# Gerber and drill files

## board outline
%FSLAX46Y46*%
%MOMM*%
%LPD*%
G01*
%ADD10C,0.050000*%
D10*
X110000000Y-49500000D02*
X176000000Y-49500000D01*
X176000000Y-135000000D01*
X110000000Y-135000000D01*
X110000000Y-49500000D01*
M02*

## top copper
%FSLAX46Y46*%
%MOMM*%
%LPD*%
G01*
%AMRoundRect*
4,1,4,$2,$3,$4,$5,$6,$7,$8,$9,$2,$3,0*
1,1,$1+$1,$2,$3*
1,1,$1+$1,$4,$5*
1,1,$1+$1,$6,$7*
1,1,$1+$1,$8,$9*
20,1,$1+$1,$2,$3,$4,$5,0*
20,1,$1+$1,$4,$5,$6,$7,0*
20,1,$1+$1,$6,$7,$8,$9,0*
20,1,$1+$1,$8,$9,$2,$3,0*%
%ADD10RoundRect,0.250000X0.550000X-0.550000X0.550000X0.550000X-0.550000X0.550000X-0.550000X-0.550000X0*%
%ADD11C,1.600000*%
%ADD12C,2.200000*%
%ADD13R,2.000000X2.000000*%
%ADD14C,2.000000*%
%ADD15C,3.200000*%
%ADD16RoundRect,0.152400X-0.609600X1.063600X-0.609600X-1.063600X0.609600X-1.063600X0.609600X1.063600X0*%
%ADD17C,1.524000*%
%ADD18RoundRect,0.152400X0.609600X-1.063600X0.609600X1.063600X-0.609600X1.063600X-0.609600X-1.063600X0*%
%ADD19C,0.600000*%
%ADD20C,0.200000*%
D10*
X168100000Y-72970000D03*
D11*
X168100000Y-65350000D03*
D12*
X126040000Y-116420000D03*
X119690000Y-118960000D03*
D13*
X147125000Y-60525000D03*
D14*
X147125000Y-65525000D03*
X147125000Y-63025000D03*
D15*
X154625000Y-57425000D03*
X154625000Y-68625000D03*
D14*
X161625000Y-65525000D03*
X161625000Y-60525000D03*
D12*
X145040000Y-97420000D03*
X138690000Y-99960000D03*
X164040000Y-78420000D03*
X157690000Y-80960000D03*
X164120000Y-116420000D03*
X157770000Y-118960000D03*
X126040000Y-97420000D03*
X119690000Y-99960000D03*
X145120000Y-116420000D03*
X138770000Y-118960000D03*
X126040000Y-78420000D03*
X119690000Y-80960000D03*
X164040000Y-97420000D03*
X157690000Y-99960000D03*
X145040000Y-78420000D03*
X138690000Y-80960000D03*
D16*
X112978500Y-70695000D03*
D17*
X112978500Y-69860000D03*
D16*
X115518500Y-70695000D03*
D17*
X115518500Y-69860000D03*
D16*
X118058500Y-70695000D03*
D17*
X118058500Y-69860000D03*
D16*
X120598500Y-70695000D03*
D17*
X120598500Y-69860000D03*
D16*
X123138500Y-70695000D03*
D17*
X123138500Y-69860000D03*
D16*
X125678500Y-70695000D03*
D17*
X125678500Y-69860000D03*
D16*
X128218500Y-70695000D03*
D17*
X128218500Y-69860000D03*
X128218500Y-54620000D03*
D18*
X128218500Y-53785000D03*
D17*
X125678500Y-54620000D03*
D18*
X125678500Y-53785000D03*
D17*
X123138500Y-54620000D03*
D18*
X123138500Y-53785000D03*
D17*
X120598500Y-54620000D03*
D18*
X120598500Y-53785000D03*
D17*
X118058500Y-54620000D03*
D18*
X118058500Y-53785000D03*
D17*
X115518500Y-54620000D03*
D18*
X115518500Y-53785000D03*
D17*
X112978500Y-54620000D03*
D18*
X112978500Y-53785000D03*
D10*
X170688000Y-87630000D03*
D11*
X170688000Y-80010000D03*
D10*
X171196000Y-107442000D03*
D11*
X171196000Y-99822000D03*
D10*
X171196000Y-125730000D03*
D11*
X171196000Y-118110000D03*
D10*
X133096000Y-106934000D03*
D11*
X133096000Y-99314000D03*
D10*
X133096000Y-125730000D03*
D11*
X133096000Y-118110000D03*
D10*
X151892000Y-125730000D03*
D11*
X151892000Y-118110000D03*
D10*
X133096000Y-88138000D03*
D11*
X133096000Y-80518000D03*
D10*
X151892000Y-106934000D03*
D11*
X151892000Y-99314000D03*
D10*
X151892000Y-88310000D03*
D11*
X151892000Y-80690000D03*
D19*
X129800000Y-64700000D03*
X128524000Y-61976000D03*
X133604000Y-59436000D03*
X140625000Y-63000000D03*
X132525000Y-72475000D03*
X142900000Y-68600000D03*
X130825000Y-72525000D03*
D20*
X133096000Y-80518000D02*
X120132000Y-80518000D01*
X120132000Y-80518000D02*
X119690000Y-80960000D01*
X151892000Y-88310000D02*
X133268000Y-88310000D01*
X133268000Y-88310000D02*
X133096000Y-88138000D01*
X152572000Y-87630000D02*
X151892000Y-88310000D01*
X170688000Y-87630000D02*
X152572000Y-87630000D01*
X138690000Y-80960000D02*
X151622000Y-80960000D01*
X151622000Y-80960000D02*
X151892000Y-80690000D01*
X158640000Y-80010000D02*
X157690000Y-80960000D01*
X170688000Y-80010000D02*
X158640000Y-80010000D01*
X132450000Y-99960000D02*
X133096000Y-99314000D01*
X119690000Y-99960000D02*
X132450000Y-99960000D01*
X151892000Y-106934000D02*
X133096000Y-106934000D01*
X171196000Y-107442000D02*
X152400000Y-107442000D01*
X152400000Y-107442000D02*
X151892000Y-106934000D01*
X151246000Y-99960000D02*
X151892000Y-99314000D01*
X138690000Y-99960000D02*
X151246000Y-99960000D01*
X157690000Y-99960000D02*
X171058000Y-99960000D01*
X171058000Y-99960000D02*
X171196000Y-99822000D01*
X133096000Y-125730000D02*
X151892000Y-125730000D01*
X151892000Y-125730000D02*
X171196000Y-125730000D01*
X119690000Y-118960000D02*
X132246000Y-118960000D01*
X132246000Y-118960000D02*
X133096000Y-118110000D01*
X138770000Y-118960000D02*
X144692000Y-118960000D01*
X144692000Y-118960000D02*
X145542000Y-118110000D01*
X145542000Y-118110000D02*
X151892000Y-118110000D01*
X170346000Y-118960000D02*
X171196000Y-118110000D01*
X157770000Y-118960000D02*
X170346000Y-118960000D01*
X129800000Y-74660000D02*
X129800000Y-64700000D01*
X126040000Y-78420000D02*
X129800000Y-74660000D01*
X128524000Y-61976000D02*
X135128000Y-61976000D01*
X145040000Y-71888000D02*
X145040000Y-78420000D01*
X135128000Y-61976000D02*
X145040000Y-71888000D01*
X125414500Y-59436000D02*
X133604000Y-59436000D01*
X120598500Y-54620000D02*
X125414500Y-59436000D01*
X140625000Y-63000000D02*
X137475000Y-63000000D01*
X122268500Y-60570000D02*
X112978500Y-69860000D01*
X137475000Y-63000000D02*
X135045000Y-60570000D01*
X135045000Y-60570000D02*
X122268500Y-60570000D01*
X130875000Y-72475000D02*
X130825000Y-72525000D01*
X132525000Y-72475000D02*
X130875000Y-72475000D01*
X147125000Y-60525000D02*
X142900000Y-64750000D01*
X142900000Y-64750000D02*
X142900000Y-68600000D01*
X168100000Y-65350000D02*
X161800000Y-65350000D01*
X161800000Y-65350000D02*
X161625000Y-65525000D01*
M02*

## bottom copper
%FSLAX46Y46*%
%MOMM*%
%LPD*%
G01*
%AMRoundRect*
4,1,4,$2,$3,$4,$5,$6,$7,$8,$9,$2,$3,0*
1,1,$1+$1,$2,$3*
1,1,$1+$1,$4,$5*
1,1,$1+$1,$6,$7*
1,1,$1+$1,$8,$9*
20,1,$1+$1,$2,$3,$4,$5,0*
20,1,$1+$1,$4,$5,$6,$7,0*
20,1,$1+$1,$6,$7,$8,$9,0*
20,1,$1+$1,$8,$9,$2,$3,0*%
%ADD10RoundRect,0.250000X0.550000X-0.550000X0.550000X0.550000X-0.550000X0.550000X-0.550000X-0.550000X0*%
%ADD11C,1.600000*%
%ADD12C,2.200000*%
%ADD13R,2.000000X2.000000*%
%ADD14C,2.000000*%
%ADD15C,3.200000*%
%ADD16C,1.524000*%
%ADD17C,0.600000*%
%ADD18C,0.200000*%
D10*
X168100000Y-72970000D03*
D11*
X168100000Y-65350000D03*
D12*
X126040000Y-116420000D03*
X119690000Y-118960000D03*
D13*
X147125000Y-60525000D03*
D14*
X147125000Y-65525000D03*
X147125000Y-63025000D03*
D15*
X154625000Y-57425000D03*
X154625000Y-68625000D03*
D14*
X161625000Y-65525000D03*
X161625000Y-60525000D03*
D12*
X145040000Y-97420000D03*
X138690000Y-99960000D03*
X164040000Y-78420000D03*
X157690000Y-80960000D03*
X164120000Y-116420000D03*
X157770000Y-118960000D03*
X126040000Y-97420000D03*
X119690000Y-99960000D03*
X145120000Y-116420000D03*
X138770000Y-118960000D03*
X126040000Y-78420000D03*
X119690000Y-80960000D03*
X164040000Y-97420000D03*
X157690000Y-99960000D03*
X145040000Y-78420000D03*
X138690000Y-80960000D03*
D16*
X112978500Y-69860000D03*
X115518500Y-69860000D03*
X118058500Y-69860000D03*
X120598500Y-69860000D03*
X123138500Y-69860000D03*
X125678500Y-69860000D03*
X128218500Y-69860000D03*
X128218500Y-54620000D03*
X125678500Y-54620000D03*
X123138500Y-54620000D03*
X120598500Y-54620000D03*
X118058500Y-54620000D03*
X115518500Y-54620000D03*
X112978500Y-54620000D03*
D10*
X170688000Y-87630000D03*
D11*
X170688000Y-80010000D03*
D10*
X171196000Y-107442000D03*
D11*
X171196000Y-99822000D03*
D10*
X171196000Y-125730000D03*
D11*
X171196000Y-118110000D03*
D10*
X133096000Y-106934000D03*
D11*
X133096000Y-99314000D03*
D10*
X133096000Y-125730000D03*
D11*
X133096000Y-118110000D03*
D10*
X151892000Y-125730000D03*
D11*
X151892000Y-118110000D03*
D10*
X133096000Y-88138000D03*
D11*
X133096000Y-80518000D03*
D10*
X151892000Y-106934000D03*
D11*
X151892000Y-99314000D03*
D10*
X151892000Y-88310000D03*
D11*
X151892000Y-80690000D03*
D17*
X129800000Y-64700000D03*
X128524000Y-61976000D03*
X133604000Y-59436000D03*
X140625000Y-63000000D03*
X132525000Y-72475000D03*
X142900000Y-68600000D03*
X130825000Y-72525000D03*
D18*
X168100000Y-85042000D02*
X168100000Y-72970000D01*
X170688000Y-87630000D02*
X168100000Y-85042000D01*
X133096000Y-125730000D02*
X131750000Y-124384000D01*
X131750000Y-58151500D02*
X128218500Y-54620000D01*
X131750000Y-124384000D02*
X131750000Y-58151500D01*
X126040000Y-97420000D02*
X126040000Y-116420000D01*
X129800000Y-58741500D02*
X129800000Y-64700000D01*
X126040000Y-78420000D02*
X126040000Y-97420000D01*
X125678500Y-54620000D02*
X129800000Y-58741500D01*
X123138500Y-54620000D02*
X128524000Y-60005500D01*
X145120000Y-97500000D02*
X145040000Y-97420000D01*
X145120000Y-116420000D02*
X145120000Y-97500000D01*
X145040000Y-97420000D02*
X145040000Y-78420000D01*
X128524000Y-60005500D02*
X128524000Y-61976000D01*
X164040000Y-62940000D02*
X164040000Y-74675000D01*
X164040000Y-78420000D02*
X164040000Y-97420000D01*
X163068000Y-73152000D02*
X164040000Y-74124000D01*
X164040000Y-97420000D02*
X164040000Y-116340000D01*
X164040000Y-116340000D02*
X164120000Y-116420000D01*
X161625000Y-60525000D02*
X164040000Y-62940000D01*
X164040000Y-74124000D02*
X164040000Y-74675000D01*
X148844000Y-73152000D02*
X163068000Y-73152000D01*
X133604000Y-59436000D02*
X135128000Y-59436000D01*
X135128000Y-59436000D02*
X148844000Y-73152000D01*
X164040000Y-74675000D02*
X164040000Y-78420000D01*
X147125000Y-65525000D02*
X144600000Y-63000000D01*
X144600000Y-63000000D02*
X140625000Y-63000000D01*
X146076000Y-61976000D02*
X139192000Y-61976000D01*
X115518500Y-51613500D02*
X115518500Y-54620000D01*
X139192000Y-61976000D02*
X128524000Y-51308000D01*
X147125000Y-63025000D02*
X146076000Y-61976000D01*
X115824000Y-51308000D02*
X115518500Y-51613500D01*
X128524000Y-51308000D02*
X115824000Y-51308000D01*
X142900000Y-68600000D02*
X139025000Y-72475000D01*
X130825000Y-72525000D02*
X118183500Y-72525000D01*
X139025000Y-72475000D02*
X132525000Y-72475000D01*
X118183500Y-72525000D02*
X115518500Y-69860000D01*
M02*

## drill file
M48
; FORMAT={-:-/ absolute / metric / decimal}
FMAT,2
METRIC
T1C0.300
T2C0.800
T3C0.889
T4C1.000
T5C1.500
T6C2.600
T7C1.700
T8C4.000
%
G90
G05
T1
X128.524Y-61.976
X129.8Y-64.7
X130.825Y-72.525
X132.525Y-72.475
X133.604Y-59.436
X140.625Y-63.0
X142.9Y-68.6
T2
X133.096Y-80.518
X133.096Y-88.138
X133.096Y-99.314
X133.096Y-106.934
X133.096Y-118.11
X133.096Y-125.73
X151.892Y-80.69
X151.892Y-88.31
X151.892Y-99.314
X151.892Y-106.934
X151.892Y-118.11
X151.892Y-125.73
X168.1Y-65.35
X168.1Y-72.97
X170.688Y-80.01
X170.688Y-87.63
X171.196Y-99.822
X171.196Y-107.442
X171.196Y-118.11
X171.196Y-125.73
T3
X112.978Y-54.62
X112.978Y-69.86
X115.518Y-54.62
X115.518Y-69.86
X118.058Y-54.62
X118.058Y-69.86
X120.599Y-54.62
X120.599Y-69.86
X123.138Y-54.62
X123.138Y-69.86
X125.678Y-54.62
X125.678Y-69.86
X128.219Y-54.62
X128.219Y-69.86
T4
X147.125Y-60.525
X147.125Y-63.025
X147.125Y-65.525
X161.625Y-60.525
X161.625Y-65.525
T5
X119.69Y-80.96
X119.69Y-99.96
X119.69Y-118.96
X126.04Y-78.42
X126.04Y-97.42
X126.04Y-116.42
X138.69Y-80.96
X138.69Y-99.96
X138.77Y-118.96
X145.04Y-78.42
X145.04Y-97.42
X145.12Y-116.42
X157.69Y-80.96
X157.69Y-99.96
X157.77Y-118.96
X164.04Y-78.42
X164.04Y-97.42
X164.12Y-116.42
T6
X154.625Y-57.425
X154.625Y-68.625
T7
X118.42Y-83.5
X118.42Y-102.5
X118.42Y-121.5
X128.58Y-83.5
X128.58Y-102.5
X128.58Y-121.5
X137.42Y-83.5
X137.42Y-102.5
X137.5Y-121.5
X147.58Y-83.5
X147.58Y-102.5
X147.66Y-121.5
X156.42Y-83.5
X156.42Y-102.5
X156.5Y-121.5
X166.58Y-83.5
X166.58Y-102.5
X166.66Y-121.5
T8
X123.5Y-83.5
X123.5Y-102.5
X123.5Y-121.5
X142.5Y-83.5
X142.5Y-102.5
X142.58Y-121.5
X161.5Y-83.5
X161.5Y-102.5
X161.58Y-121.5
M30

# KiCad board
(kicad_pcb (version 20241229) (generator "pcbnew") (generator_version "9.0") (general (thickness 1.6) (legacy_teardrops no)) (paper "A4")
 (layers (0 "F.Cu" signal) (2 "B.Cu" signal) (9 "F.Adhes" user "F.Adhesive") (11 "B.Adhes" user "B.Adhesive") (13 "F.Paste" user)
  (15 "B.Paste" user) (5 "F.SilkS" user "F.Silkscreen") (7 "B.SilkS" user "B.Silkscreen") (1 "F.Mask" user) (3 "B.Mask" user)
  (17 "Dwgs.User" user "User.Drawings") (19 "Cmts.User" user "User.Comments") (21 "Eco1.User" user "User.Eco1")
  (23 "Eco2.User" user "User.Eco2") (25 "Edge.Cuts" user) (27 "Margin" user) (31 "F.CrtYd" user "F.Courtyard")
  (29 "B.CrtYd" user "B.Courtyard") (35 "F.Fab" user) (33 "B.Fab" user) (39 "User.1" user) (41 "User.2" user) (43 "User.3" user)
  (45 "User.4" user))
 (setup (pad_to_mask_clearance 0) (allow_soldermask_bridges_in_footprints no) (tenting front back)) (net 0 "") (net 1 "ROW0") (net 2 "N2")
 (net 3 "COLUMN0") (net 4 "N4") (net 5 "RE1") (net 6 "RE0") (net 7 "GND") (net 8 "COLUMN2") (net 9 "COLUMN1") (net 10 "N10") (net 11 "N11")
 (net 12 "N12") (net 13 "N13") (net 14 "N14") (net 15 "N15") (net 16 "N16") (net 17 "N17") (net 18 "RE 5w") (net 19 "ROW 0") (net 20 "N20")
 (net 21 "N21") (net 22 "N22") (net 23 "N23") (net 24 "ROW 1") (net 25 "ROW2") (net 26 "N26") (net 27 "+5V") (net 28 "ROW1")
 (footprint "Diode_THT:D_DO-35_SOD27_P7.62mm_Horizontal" (layer "F.Cu") (at 168.1 72.97 90)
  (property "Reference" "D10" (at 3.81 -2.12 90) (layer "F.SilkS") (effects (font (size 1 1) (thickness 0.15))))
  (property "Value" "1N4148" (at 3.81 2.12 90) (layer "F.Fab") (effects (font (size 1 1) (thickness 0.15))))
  (pad "1" thru_hole roundrect (at 0 0 90) (size 1.6 1.6) (drill 0.8) (layers "*.Cu" "*.Mask") (remove_unused_layers no)
   (roundrect_rratio 0.15625) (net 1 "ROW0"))
  (pad "2" thru_hole circle (at 7.62 0 90) (size 1.6 1.6) (drill 0.8) (layers "*.Cu" "*.Mask") (remove_unused_layers no) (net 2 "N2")))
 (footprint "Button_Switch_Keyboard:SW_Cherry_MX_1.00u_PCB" (layer "F.Cu") (at 126.04 116.42)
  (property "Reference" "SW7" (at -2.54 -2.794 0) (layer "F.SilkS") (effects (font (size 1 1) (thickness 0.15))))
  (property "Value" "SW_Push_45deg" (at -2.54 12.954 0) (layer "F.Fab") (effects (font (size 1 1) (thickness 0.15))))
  (pad "" np_thru_hole circle (at -7.62 5.08) (size 1.7 1.7) (drill 1.7) (layers "*.Cu" "*.Mask"))
  (pad "" np_thru_hole circle (at -2.54 5.08) (size 4 4) (drill 4) (layers "*.Cu" "*.Mask"))
  (pad "" np_thru_hole circle (at 2.54 5.08) (size 1.7 1.7) (drill 1.7) (layers "*.Cu" "*.Mask"))
  (pad "1" thru_hole circle (at 0 0) (size 2.2 2.2) (drill 1.5) (layers "*.Cu" "*.Mask") (remove_unused_layers no) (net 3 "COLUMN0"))
  (pad "2" thru_hole circle (at -6.35 2.54) (size 2.2 2.2) (drill 1.5) (layers "*.Cu" "*.Mask") (remove_unused_layers no) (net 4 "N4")))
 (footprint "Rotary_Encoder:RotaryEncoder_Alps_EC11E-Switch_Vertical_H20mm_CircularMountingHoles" (layer "F.Cu") (at 147.125 60.525)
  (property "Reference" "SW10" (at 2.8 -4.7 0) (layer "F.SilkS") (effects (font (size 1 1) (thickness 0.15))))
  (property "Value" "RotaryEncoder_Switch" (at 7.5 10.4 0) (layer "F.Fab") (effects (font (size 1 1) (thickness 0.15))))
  (pad "A" thru_hole rect (at 0 0) (size 2 2) (drill 1) (layers "*.Cu" "*.Mask") (remove_unused_layers no) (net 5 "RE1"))
  (pad "B" thru_hole circle (at 0 5) (size 2 2) (drill 1) (layers "*.Cu" "*.Mask") (remove_unused_layers no) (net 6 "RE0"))
  (pad "C" thru_hole circle (at 0 2.5) (size 2 2) (drill 1) (layers "*.Cu" "*.Mask") (remove_unused_layers no) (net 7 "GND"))
  (pad "MP" thru_hole circle (at 7.5 -3.1) (size 3.2 3.2) (drill 2.6) (layers "*.Cu" "*.Mask") (remove_unused_layers no))
  (pad "MP" thru_hole circle (at 7.5 8.1) (size 3.2 3.2) (drill 2.6) (layers "*.Cu" "*.Mask") (remove_unused_layers no))
  (pad "S1" thru_hole circle (at 14.5 5) (size 2 2) (drill 1) (layers "*.Cu" "*.Mask") (remove_unused_layers no) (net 2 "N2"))
  (pad "S2" thru_hole circle (at 14.5 0) (size 2 2) (drill 1) (layers "*.Cu" "*.Mask") (remove_unused_layers no) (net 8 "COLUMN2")))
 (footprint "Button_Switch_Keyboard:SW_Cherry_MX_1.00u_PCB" (layer "F.Cu") (at 145.04 97.42)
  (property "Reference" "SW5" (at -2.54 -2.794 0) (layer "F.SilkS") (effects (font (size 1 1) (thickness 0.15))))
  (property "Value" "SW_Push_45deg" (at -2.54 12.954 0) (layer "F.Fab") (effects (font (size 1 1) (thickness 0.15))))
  (pad "" np_thru_hole circle (at -7.62 5.08) (size 1.7 1.7) (drill 1.7) (layers "*.Cu" "*.Mask"))
  (pad "" np_thru_hole circle (at -2.54 5.08) (size 4 4) (drill 4) (layers "*.Cu" "*.Mask"))
  (pad "" np_thru_hole circle (at 2.54 5.08) (size 1.7 1.7) (drill 1.7) (layers "*.Cu" "*.Mask"))
  (pad "1" thru_hole circle (at 0 0) (size 2.2 2.2) (drill 1.5) (layers "*.Cu" "*.Mask") (remove_unused_layers no) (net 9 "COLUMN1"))
  (pad "2" thru_hole circle (at -6.35 2.54) (size 2.2 2.2) (drill 1.5) (layers "*.Cu" "*.Mask") (remove_unused_layers no) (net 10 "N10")))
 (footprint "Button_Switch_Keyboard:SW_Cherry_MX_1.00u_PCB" (layer "F.Cu") (at 164.04 78.42)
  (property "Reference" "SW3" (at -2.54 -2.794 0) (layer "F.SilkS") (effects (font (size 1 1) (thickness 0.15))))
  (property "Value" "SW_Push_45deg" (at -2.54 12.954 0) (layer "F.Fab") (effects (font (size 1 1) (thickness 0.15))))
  (pad "" np_thru_hole circle (at -7.62 5.08) (size 1.7 1.7) (drill 1.7) (layers "*.Cu" "*.Mask"))
  (pad "" np_thru_hole circle (at -2.54 5.08) (size 4 4) (drill 4) (layers "*.Cu" "*.Mask"))
  (pad "" np_thru_hole circle (at 2.54 5.08) (size 1.7 1.7) (drill 1.7) (layers "*.Cu" "*.Mask"))
  (pad "1" thru_hole circle (at 0 0) (size 2.2 2.2) (drill 1.5) (layers "*.Cu" "*.Mask") (remove_unused_layers no) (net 8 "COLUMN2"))
  (pad "2" thru_hole circle (at -6.35 2.54) (size 2.2 2.2) (drill 1.5) (layers "*.Cu" "*.Mask") (remove_unused_layers no) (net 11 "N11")))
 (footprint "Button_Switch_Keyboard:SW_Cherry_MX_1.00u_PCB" (layer "F.Cu") (at 164.12 116.42)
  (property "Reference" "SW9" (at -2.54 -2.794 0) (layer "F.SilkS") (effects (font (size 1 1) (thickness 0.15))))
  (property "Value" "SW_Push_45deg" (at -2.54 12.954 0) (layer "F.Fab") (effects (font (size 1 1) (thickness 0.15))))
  (pad "" np_thru_hole circle (at -7.62 5.08) (size 1.7 1.7) (drill 1.7) (layers "*.Cu" "*.Mask"))
  (pad "" np_thru_hole circle (at -2.54 5.08) (size 4 4) (drill 4) (layers "*.Cu" "*.Mask"))
  (pad "" np_thru_hole circle (at 2.54 5.08) (size 1.7 1.7) (drill 1.7) (layers "*.Cu" "*.Mask"))
  (pad "1" thru_hole circle (at 0 0) (size 2.2 2.2) (drill 1.5) (layers "*.Cu" "*.Mask") (remove_unused_layers no) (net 8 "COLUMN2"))
  (pad "2" thru_hole circle (at -6.35 2.54) (size 2.2 2.2) (drill 1.5) (layers "*.Cu" "*.Mask") (remove_unused_layers no) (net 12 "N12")))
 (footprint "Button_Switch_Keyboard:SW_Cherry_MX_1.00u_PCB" (layer "F.Cu") (at 126.04 97.42)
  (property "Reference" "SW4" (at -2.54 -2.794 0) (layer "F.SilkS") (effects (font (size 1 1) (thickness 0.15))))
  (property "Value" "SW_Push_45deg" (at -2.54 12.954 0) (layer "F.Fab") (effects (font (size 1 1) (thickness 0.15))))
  (pad "" np_thru_hole circle (at -7.62 5.08) (size 1.7 1.7) (drill 1.7) (layers "*.Cu" "*.Mask"))
  (pad "" np_thru_hole circle (at -2.54 5.08) (size 4 4) (drill 4) (layers "*.Cu" "*.Mask"))
  (pad "" np_thru_hole circle (at 2.54 5.08) (size 1.7 1.7) (drill 1.7) (layers "*.Cu" "*.Mask"))
  (pad "1" thru_hole circle (at 0 0) (size 2.2 2.2) (drill 1.5) (layers "*.Cu" "*.Mask") (remove_unused_layers no) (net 3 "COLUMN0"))
  (pad "2" thru_hole circle (at -6.35 2.54) (size 2.2 2.2) (drill 1.5) (layers "*.Cu" "*.Mask") (remove_unused_layers no) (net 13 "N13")))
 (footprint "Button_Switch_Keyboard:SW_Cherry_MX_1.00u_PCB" (layer "F.Cu") (at 145.12 116.42)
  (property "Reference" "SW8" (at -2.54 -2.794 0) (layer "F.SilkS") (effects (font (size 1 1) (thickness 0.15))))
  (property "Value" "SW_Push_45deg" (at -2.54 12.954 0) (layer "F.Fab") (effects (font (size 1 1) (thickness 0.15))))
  (pad "" np_thru_hole circle (at -7.62 5.08) (size 1.7 1.7) (drill 1.7) (layers "*.Cu" "*.Mask"))
  (pad "" np_thru_hole circle (at -2.54 5.08) (size 4 4) (drill 4) (layers "*.Cu" "*.Mask"))
  (pad "" np_thru_hole circle (at 2.54 5.08) (size 1.7 1.7) (drill 1.7) (layers "*.Cu" "*.Mask"))
  (pad "1" thru_hole circle (at 0 0) (size 2.2 2.2) (drill 1.5) (layers "*.Cu" "*.Mask") (remove_unused_layers no) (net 9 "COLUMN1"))
  (pad "2" thru_hole circle (at -6.35 2.54) (size 2.2 2.2) (drill 1.5) (layers "*.Cu" "*.Mask") (remove_unused_layers no) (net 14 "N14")))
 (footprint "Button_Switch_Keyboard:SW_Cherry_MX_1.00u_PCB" (layer "F.Cu") (at 126.04 78.42)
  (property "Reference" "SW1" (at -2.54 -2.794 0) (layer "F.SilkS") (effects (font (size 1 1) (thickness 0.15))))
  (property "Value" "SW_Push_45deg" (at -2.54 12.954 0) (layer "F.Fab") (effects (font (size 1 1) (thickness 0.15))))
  (pad "" np_thru_hole circle (at -7.62 5.08) (size 1.7 1.7) (drill 1.7) (layers "*.Cu" "*.Mask"))
  (pad "" np_thru_hole circle (at -2.54 5.08) (size 4 4) (drill 4) (layers "*.Cu" "*.Mask"))
  (pad "" np_thru_hole circle (at 2.54 5.08) (size 1.7 1.7) (drill 1.7) (layers "*.Cu" "*.Mask"))
  (pad "1" thru_hole circle (at 0 0) (size 2.2 2.2) (drill 1.5) (layers "*.Cu" "*.Mask") (remove_unused_layers no) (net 3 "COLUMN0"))
  (pad "2" thru_hole circle (at -6.35 2.54) (size 2.2 2.2) (drill 1.5) (layers "*.Cu" "*.Mask") (remove_unused_layers no) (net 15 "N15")))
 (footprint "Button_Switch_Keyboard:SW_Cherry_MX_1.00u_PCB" (layer "F.Cu") (at 164.04 97.42)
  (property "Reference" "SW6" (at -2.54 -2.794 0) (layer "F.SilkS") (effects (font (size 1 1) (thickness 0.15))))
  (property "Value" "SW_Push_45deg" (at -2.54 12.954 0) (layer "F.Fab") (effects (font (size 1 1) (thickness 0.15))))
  (pad "" np_thru_hole circle (at -7.62 5.08) (size 1.7 1.7) (drill 1.7) (layers "*.Cu" "*.Mask"))
  (pad "" np_thru_hole circle (at -2.54 5.08) (size 4 4) (drill 4) (layers "*.Cu" "*.Mask"))
  (pad "" np_thru_hole circle (at 2.54 5.08) (size 1.7 1.7) (drill 1.7) (layers "*.Cu" "*.Mask"))
  (pad "1" thru_hole circle (at 0 0) (size 2.2 2.2) (drill 1.5) (layers "*.Cu" "*.Mask") (remove_unused_layers no) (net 8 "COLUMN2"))
  (pad "2" thru_hole circle (at -6.35 2.54) (size 2.2 2.2) (drill 1.5) (layers "*.Cu" "*.Mask") (remove_unused_layers no) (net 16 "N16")))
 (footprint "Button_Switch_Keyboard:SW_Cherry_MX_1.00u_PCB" (layer "F.Cu") (at 145.04 78.42)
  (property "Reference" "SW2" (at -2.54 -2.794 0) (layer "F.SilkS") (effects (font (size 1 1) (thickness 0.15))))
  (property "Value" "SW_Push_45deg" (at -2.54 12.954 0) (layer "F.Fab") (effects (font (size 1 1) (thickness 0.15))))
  (pad "" np_thru_hole circle (at -7.62 5.08) (size 1.7 1.7) (drill 1.7) (layers "*.Cu" "*.Mask"))
  (pad "" np_thru_hole circle (at -2.54 5.08) (size 4 4) (drill 4) (layers "*.Cu" "*.Mask"))
  (pad "" np_thru_hole circle (at 2.54 5.08) (size 1.7 1.7) (drill 1.7) (layers "*.Cu" "*.Mask"))
  (pad "1" thru_hole circle (at 0 0) (size 2.2 2.2) (drill 1.5) (layers "*.Cu" "*.Mask") (remove_unused_layers no) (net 9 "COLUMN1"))
  (pad "2" thru_hole circle (at -6.35 2.54) (size 2.2 2.2) (drill 1.5) (layers "*.Cu" "*.Mask") (remove_unused_layers no) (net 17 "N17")))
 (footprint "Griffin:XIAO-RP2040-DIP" (layer "F.Cu") (at 120.5985 62.24 90)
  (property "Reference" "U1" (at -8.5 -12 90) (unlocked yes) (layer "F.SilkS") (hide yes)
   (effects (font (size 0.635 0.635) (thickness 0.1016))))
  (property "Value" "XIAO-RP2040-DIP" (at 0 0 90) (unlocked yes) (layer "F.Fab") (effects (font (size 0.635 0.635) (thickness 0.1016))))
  (pad "1" smd roundrect (at -8.455 -7.62 270) (size 2.432 1.524) (layers "F.Cu" "F.Mask") (roundrect_rratio 0.1) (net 6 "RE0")
   (thermal_bridge_angle 45))
  (pad "1" thru_hole circle (at -7.62 -7.62 270) (size 1.524 1.524) (drill 0.889) (layers "*.Cu" "*.Mask") (remove_unused_layers no)
   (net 6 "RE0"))
  (pad "2" smd roundrect (at -8.455 -5.08 270) (size 2.432 1.524) (layers "F.Cu" "F.Mask") (roundrect_rratio 0.1) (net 5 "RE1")
   (thermal_bridge_angle 45))
  (pad "2" thru_hole circle (at -7.62 -5.08 270) (size 1.524 1.524) (drill 0.889) (layers "*.Cu" "*.Mask") (remove_unused_layers no)
   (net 5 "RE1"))
  (pad "3" smd roundrect (at -8.455 -2.54 270) (size 2.432 1.524) (layers "F.Cu" "F.Mask") (roundrect_rratio 0.1) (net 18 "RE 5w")
   (thermal_bridge_angle 45))
  (pad "3" thru_hole circle (at -7.62 -2.54 270) (size 1.524 1.524) (drill 0.889) (layers "*.Cu" "*.Mask") (remove_unused_layers no)
   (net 18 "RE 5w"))
  (pad "4" smd roundrect (at -8.455 0 270) (size 2.432 1.524) (layers "F.Cu" "F.Mask") (roundrect_rratio 0.1) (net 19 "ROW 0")
   (thermal_bridge_angle 45))
  (pad "4" thru_hole circle (at -7.62 0 270) (size 1.524 1.524) (drill 0.889) (layers "*.Cu" "*.Mask") (remove_unused_layers no)
   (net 19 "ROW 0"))
  (pad "5" smd roundrect (at -8.455 2.54 270) (size 2.432 1.524) (layers "F.Cu" "F.Mask") (roundrect_rratio 0.1) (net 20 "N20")
   (thermal_bridge_angle 45))
  (pad "5" thru_hole circle (at -7.62 2.54 270) (size 1.524 1.524) (drill 0.889) (layers "*.Cu" "*.Mask") (remove_unused_layers no)
   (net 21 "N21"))
  (pad "6" smd roundrect (at -8.455 5.08 270) (size 2.432 1.524) (layers "F.Cu" "F.Mask") (roundrect_rratio 0.1) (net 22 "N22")
   (thermal_bridge_angle 45))
  (pad "6" thru_hole circle (at -7.62 5.08 270) (size 1.524 1.524) (drill 0.889) (layers "*.Cu" "*.Mask") (remove_unused_layers no)
   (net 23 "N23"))
  (pad "7" smd roundrect (at -8.455 7.62 270) (size 2.432 1.524) (layers "F.Cu" "F.Mask") (roundrect_rratio 0.1) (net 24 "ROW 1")
   (thermal_bridge_angle 45))
  (pad "7" thru_hole circle (at -7.62 7.62 270) (size 1.524 1.524) (drill 0.889) (layers "*.Cu" "*.Mask") (remove_unused_layers no)
   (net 24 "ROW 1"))
  (pad "8" thru_hole circle (at 7.62 7.62 90) (size 1.524 1.524) (drill 0.889) (layers "*.Cu" "*.Mask") (remove_unused_layers no)
   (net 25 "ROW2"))
  (pad "8" smd roundrect (at 8.455 7.62 90) (size 2.432 1.524) (layers "F.Cu" "F.Mask") (roundrect_rratio 0.1) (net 25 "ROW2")
   (thermal_bridge_angle 45))
  (pad "9" thru_hole circle (at 7.62 5.08 90) (size 1.524 1.524) (drill 0.889) (layers "*.Cu" "*.Mask") (remove_unused_layers no)
   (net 3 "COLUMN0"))
  (pad "9" smd roundrect (at 8.455 5.08 90) (size 2.432 1.524) (layers "F.Cu" "F.Mask") (roundrect_rratio 0.1) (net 3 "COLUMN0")
   (thermal_bridge_angle 45))
  (pad "10" thru_hole circle (at 7.62 2.54 90) (size 1.524 1.524) (drill 0.889) (layers "*.Cu" "*.Mask") (remove_unused_layers no)
   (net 9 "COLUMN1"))
  (pad "10" smd roundrect (at 8.455 2.54 90) (size 2.432 1.524) (layers "F.Cu" "F.Mask") (roundrect_rratio 0.1) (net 9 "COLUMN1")
   (thermal_bridge_angle 45))
  (pad "11" thru_hole circle (at 7.62 0 90) (size 1.524 1.524) (drill 0.889) (layers "*.Cu" "*.Mask") (remove_unused_layers no)
   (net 8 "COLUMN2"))
  (pad "11" smd roundrect (at 8.455 0 90) (size 2.432 1.524) (layers "F.Cu" "F.Mask") (roundrect_rratio 0.1) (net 8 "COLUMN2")
   (thermal_bridge_angle 45))
  (pad "12" thru_hole circle (at 7.62 -2.54 90) (size 1.524 1.524) (drill 0.889) (layers "*.Cu" "*.Mask") (remove_unused_layers no)
   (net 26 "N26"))
  (pad "12" smd roundrect (at 8.455 -2.54 90) (size 2.432 1.524) (layers "F.Cu" "F.Mask") (roundrect_rratio 0.1) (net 26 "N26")
   (thermal_bridge_angle 45))
  (pad "13" thru_hole circle (at 7.62 -5.08 90) (size 1.524 1.524) (drill 0.889) (layers "*.Cu" "*.Mask") (remove_unused_layers no)
   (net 7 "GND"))
  (pad "13" smd roundrect (at 8.455 -5.08 90) (size 2.432 1.524) (layers "F.Cu" "F.Mask") (roundrect_rratio 0.1) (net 7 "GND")
   (thermal_bridge_angle 45))
  (pad "14" thru_hole circle (at 7.62 -7.62 90) (size 1.524 1.524) (drill 0.889) (layers "*.Cu" "*.Mask") (remove_unused_layers no)
   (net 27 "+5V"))
  (pad "14" smd roundrect (at 8.455 -7.62 90) (size 2.432 1.524) (layers "F.Cu" "F.Mask") (roundrect_rratio 0.1) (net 27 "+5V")
   (thermal_bridge_angle 45)))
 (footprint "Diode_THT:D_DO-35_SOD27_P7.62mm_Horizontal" (layer "B.Cu") (at 170.688 87.63 90)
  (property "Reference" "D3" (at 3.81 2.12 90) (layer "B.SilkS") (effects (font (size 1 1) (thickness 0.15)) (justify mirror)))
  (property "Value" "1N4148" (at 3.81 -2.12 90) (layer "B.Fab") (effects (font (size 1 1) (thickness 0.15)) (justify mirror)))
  (pad "1" thru_hole roundrect (at 0 0 90) (size 1.6 1.6) (drill 0.8) (layers "*.Cu" "*.Mask") (remove_unused_layers no)
   (roundrect_rratio 0.15625) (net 1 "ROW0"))
  (pad "2" thru_hole circle (at 7.62 0 90) (size 1.6 1.6) (drill 0.8) (layers "*.Cu" "*.Mask") (remove_unused_layers no) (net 11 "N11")))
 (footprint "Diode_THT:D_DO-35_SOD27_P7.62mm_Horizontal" (layer "B.Cu") (at 171.196 107.442 90)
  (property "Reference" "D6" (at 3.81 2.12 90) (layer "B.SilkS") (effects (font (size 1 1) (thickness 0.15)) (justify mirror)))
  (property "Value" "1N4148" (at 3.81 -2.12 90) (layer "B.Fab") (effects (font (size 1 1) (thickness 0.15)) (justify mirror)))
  (pad "1" thru_hole roundrect (at 0 0 90) (size 1.6 1.6) (drill 0.8) (layers "*.Cu" "*.Mask") (remove_unused_layers no)
   (roundrect_rratio 0.15625) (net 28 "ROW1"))
  (pad "2" thru_hole circle (at 7.62 0 90) (size 1.6 1.6) (drill 0.8) (layers "*.Cu" "*.Mask") (remove_unused_layers no) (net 16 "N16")))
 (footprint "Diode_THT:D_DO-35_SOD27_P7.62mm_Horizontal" (layer "B.Cu") (at 171.196 125.73 90)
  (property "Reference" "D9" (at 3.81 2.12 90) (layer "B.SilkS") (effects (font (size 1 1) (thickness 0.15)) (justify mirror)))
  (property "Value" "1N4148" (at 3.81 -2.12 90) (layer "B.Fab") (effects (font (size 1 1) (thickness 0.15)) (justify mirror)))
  (pad "1" thru_hole roundrect (at 0 0 90) (size 1.6 1.6) (drill 0.8) (layers "*.Cu" "*.Mask") (remove_unused_layers no)
   (roundrect_rratio 0.15625) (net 25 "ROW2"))
  (pad "2" thru_hole circle (at 7.62 0 90) (size 1.6 1.6) (drill 0.8) (layers "*.Cu" "*.Mask") (remove_unused_layers no) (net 12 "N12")))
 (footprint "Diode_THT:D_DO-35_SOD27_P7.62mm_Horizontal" (layer "B.Cu") (at 133.096 106.934 90)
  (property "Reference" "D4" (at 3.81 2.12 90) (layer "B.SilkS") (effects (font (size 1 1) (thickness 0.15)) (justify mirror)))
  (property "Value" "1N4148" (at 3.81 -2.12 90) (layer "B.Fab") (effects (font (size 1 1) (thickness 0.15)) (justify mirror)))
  (pad "1" thru_hole roundrect (at 0 0 90) (size 1.6 1.6) (drill 0.8) (layers "*.Cu" "*.Mask") (remove_unused_layers no)
   (roundrect_rratio 0.15625) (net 28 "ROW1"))
  (pad "2" thru_hole circle (at 7.62 0 90) (size 1.6 1.6) (drill 0.8) (layers "*.Cu" "*.Mask") (remove_unused_layers no) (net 13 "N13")))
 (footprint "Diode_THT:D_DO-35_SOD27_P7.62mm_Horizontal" (layer "B.Cu") (at 133.096 125.73 90)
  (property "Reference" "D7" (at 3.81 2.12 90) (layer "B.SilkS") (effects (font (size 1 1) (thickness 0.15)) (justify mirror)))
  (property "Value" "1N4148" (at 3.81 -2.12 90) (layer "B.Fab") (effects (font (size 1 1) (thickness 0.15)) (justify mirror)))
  (pad "1" thru_hole roundrect (at 0 0 90) (size 1.6 1.6) (drill 0.8) (layers "*.Cu" "*.Mask") (remove_unused_layers no)
   (roundrect_rratio 0.15625) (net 25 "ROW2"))
  (pad "2" thru_hole circle (at 7.62 0 90) (size 1.6 1.6) (drill 0.8) (layers "*.Cu" "*.Mask") (remove_unused_layers no) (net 4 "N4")))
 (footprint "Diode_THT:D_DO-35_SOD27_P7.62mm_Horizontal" (layer "B.Cu") (at 151.892 125.73 90)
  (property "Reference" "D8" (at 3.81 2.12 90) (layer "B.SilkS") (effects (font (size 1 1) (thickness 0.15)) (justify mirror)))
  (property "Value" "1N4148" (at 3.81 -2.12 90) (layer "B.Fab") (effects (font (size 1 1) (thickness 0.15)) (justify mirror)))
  (pad "1" thru_hole roundrect (at 0 0 90) (size 1.6 1.6) (drill 0.8) (layers "*.Cu" "*.Mask") (remove_unused_layers no)
   (roundrect_rratio 0.15625) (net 25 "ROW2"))
  (pad "2" thru_hole circle (at 7.62 0 90) (size 1.6 1.6) (drill 0.8) (layers "*.Cu" "*.Mask") (remove_unused_layers no) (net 14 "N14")))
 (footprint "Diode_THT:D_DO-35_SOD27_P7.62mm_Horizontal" (layer "B.Cu") (at 133.096 88.138 90)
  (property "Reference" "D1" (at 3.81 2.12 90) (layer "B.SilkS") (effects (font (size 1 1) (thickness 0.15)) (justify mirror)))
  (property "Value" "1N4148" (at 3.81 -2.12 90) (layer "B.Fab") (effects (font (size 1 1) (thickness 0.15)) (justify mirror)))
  (pad "1" thru_hole roundrect (at 0 0 90) (size 1.6 1.6) (drill 0.8) (layers "*.Cu" "*.Mask") (remove_unused_layers no)
   (roundrect_rratio 0.15625) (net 1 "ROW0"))
  (pad "2" thru_hole circle (at 7.62 0 90) (size 1.6 1.6) (drill 0.8) (layers "*.Cu" "*.Mask") (remove_unused_layers no) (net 15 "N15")))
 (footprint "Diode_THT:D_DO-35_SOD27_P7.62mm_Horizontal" (layer "B.Cu") (at 151.892 106.934 90)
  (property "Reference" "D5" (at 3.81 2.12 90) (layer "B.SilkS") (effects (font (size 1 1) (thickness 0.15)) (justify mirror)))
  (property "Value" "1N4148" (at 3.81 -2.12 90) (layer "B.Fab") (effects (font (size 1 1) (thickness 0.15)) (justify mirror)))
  (pad "1" thru_hole roundrect (at 0 0 90) (size 1.6 1.6) (drill 0.8) (layers "*.Cu" "*.Mask") (remove_unused_layers no)
   (roundrect_rratio 0.15625) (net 28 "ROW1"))
  (pad "2" thru_hole circle (at 7.62 0 90) (size 1.6 1.6) (drill 0.8) (layers "*.Cu" "*.Mask") (remove_unused_layers no) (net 10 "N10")))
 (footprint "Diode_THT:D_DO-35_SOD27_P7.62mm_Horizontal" (layer "B.Cu") (at 151.892 88.31 90)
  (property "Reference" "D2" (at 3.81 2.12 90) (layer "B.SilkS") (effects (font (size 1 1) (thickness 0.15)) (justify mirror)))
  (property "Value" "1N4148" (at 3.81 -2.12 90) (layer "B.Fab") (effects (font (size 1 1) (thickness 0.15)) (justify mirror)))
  (pad "1" thru_hole roundrect (at 0 0 90) (size 1.6 1.6) (drill 0.8) (layers "*.Cu" "*.Mask") (remove_unused_layers no)
   (roundrect_rratio 0.15625) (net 1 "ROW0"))
  (pad "2" thru_hole circle (at 7.62 0 90) (size 1.6 1.6) (drill 0.8) (layers "*.Cu" "*.Mask") (remove_unused_layers no) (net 17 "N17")))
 (gr_rect (start 110 49.5) (end 176 135) (stroke (width 0.05) (type default)) (fill no) (layer "Edge.Cuts"))
 (segment (start 133.096 80.518) (end 120.132 80.518) (width 0.2) (layer "F.Cu") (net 15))
 (segment (start 120.132 80.518) (end 119.69 80.96) (width 0.2) (layer "F.Cu") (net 15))
 (segment (start 151.892 88.31) (end 133.268 88.31) (width 0.2) (layer "F.Cu") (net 1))
 (segment (start 133.268 88.31) (end 133.096 88.138) (width 0.2) (layer "F.Cu") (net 1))
 (segment (start 152.572 87.63) (end 151.892 88.31) (width 0.2) (layer "F.Cu") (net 1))
 (segment (start 170.688 87.63) (end 152.572 87.63) (width 0.2) (layer "F.Cu") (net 1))
 (segment (start 168.1 85.042) (end 168.1 72.97) (width 0.2) (layer "B.Cu") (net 1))
 (segment (start 170.688 87.63) (end 168.1 85.042) (width 0.2) (layer "B.Cu") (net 1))
 (segment (start 138.69 80.96) (end 151.622 80.96) (width 0.2) (layer "F.Cu") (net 17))
 (segment (start 151.622 80.96) (end 151.892 80.69) (width 0.2) (layer "F.Cu") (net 17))
 (segment (start 158.64 80.01) (end 157.69 80.96) (width 0.2) (layer "F.Cu") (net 11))
 (segment (start 170.688 80.01) (end 158.64 80.01) (width 0.2) (layer "F.Cu") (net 11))
 (segment (start 132.45 99.96) (end 133.096 99.314) (width 0.2) (layer "F.Cu") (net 13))
 (segment (start 119.69 99.96) (end 132.45 99.96) (width 0.2) (layer "F.Cu") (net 13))
 (segment (start 151.892 106.934) (end 133.096 106.934) (width 0.2) (layer "F.Cu") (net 28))
 (segment (start 171.196 107.442) (end 152.4 107.442) (width 0.2) (layer "F.Cu") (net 28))
 (segment (start 152.4 107.442) (end 151.892 106.934) (width 0.2) (layer "F.Cu") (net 28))
 (segment (start 151.246 99.96) (end 151.892 99.314) (width 0.2) (layer "F.Cu") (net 10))
 (segment (start 138.69 99.96) (end 151.246 99.96) (width 0.2) (layer "F.Cu") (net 10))
 (segment (start 157.69 99.96) (end 171.058 99.96) (width 0.2) (layer "F.Cu") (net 16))
 (segment (start 171.058 99.96) (end 171.196 99.822) (width 0.2) (layer "F.Cu") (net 16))
 (segment (start 133.096 125.73) (end 151.892 125.73) (width 0.2) (layer "F.Cu") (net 25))
 (segment (start 151.892 125.73) (end 171.196 125.73) (width 0.2) (layer "F.Cu") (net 25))
 (segment (start 133.096 125.73) (end 131.75 124.384) (width 0.2) (layer "B.Cu") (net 25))
 (segment (start 131.75 58.1515) (end 128.2185 54.62) (width 0.2) (layer "B.Cu") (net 25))
 (segment (start 131.75 124.384) (end 131.75 58.1515) (width 0.2) (layer "B.Cu") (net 25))
 (segment (start 119.69 118.96) (end 132.246 118.96) (width 0.2) (layer "F.Cu") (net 4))
 (segment (start 132.246 118.96) (end 133.096 118.11) (width 0.2) (layer "F.Cu") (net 4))
 (segment (start 138.77 118.96) (end 144.692 118.96) (width 0.2) (layer "F.Cu") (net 14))
 (segment (start 144.692 118.96) (end 145.542 118.11) (width 0.2) (layer "F.Cu") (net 14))
 (segment (start 145.542 118.11) (end 151.892 118.11) (width 0.2) (layer "F.Cu") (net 14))
 (segment (start 170.346 118.96) (end 171.196 118.11) (width 0.2) (layer "F.Cu") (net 12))
 (segment (start 157.77 118.96) (end 170.346 118.96) (width 0.2) (layer "F.Cu") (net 12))
 (segment (start 129.8 74.66) (end 129.8 64.7) (width 0.2) (layer "F.Cu") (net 3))
 (segment (start 126.04 78.42) (end 129.8 74.66) (width 0.2) (layer "F.Cu") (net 3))
 (via (at 129.8 64.7) (size 0.6) (drill 0.3) (layers "F.Cu" "B.Cu") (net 3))
 (segment (start 126.04 97.42) (end 126.04 116.42) (width 0.2) (layer "B.Cu") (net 3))
 (segment (start 129.8 58.7415) (end 129.8 64.7) (width 0.2) (layer "B.Cu") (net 3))
 (segment (start 126.04 78.42) (end 126.04 97.42) (width 0.2) (layer "B.Cu") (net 3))
 (segment (start 125.6785 54.62) (end 129.8 58.7415) (width 0.2) (layer "B.Cu") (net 3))
 (segment (start 128.524 61.976) (end 135.128 61.976) (width 0.2) (layer "F.Cu") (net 9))
 (segment (start 145.04 71.888) (end 145.04 78.42) (width 0.2) (layer "F.Cu") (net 9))
 (segment (start 135.128 61.976) (end 145.04 71.888) (width 0.2) (layer "F.Cu") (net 9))
 (via (at 128.524 61.976) (size 0.6) (drill 0.3) (layers "F.Cu" "B.Cu") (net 9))
 (segment (start 123.1385 54.62) (end 128.524 60.0055) (width 0.2) (layer "B.Cu") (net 9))
 (segment (start 145.12 97.5) (end 145.04 97.42) (width 0.2) (layer "B.Cu") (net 9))
 (segment (start 145.12 116.42) (end 145.12 97.5) (width 0.2) (layer "B.Cu") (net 9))
 (segment (start 145.04 97.42) (end 145.04 78.42) (width 0.2) (layer "B.Cu") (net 9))
 (segment (start 128.524 60.0055) (end 128.524 61.976) (width 0.2) (layer "B.Cu") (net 9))
 (segment (start 125.4145 59.436) (end 133.604 59.436) (width 0.2) (layer "F.Cu") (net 8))
 (segment (start 120.5985 54.62) (end 125.4145 59.436) (width 0.2) (layer "F.Cu") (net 8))
 (via (at 133.604 59.436) (size 0.6) (drill 0.3) (layers "F.Cu" "B.Cu") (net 8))
 (segment (start 164.04 62.94) (end 164.04 74.675) (width 0.2) (layer "B.Cu") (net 8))
 (segment (start 164.04 78.42) (end 164.04 97.42) (width 0.2) (layer "B.Cu") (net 8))
 (segment (start 163.068 73.152) (end 164.04 74.124) (width 0.2) (layer "B.Cu") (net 8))
 (segment (start 164.04 97.42) (end 164.04 116.34) (width 0.2) (layer "B.Cu") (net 8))
 (segment (start 164.04 116.34) (end 164.12 116.42) (width 0.2) (layer "B.Cu") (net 8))
 (segment (start 161.625 60.525) (end 164.04 62.94) (width 0.2) (layer "B.Cu") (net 8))
 (segment (start 164.04 74.124) (end 164.04 74.675) (width 0.2) (layer "B.Cu") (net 8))
 (segment (start 148.844 73.152) (end 163.068 73.152) (width 0.2) (layer "B.Cu") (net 8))
 (segment (start 133.604 59.436) (end 135.128 59.436) (width 0.2) (layer "B.Cu") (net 8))
 (segment (start 135.128 59.436) (end 148.844 73.152) (width 0.2) (layer "B.Cu") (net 8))
 (segment (start 164.04 74.675) (end 164.04 78.42) (width 0.2) (layer "B.Cu") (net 8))
 (segment (start 140.625 63) (end 137.475 63) (width 0.2) (layer "F.Cu") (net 6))
 (segment (start 122.2685 60.57) (end 112.9785 69.86) (width 0.2) (layer "F.Cu") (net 6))
 (segment (start 137.475 63) (end 135.045 60.57) (width 0.2) (layer "F.Cu") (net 6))
 (segment (start 135.045 60.57) (end 122.2685 60.57) (width 0.2) (layer "F.Cu") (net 6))
 (via (at 140.625 63) (size 0.6) (drill 0.3) (layers "F.Cu" "B.Cu") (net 6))
 (segment (start 147.125 65.525) (end 144.6 63) (width 0.2) (layer "B.Cu") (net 6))
 (segment (start 144.6 63) (end 140.625 63) (width 0.2) (layer "B.Cu") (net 6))
 (segment (start 146.076 61.976) (end 139.192 61.976) (width 0.2) (layer "B.Cu") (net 7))
 (segment (start 115.5185 51.6135) (end 115.5185 54.62) (width 0.2) (layer "B.Cu") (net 7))
 (segment (start 139.192 61.976) (end 128.524 51.308) (width 0.2) (layer "B.Cu") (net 7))
 (segment (start 147.125 63.025) (end 146.076 61.976) (width 0.2) (layer "B.Cu") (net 7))
 (segment (start 115.824 51.308) (end 115.5185 51.6135) (width 0.2) (layer "B.Cu") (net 7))
 (segment (start 128.524 51.308) (end 115.824 51.308) (width 0.2) (layer "B.Cu") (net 7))
 (segment (start 130.875 72.475) (end 130.825 72.525) (width 0.2) (layer "F.Cu") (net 5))
 (segment (start 132.525 72.475) (end 130.875 72.475) (width 0.2) (layer "F.Cu") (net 5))
 (segment (start 147.125 60.525) (end 142.9 64.75) (width 0.2) (layer "F.Cu") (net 5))
 (segment (start 142.9 64.75) (end 142.9 68.6) (width 0.2) (layer "F.Cu") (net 5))
 (via (at 132.525 72.475) (size 0.6) (drill 0.3) (layers "F.Cu" "B.Cu") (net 5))
 (via (at 142.9 68.6) (size 0.6) (drill 0.3) (layers "F.Cu" "B.Cu") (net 5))
 (via (at 130.825 72.525) (size 0.6) (drill 0.3) (layers "F.Cu" "B.Cu") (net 5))
 (segment (start 142.9 68.6) (end 139.025 72.475) (width 0.2) (layer "B.Cu") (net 5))
 (segment (start 130.825 72.525) (end 118.1835 72.525) (width 0.2) (layer "B.Cu") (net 5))
 (segment (start 139.025 72.475) (end 132.525 72.475) (width 0.2) (layer "B.Cu") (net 5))
 (segment (start 118.1835 72.525) (end 115.5185 69.86) (width 0.2) (layer "B.Cu") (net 5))
 (segment (start 168.1 65.35) (end 161.8 65.35) (width 0.2) (layer "F.Cu") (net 2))
 (segment (start 161.8 65.35) (end 161.625 65.525) (width 0.2) (layer "F.Cu") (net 2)))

